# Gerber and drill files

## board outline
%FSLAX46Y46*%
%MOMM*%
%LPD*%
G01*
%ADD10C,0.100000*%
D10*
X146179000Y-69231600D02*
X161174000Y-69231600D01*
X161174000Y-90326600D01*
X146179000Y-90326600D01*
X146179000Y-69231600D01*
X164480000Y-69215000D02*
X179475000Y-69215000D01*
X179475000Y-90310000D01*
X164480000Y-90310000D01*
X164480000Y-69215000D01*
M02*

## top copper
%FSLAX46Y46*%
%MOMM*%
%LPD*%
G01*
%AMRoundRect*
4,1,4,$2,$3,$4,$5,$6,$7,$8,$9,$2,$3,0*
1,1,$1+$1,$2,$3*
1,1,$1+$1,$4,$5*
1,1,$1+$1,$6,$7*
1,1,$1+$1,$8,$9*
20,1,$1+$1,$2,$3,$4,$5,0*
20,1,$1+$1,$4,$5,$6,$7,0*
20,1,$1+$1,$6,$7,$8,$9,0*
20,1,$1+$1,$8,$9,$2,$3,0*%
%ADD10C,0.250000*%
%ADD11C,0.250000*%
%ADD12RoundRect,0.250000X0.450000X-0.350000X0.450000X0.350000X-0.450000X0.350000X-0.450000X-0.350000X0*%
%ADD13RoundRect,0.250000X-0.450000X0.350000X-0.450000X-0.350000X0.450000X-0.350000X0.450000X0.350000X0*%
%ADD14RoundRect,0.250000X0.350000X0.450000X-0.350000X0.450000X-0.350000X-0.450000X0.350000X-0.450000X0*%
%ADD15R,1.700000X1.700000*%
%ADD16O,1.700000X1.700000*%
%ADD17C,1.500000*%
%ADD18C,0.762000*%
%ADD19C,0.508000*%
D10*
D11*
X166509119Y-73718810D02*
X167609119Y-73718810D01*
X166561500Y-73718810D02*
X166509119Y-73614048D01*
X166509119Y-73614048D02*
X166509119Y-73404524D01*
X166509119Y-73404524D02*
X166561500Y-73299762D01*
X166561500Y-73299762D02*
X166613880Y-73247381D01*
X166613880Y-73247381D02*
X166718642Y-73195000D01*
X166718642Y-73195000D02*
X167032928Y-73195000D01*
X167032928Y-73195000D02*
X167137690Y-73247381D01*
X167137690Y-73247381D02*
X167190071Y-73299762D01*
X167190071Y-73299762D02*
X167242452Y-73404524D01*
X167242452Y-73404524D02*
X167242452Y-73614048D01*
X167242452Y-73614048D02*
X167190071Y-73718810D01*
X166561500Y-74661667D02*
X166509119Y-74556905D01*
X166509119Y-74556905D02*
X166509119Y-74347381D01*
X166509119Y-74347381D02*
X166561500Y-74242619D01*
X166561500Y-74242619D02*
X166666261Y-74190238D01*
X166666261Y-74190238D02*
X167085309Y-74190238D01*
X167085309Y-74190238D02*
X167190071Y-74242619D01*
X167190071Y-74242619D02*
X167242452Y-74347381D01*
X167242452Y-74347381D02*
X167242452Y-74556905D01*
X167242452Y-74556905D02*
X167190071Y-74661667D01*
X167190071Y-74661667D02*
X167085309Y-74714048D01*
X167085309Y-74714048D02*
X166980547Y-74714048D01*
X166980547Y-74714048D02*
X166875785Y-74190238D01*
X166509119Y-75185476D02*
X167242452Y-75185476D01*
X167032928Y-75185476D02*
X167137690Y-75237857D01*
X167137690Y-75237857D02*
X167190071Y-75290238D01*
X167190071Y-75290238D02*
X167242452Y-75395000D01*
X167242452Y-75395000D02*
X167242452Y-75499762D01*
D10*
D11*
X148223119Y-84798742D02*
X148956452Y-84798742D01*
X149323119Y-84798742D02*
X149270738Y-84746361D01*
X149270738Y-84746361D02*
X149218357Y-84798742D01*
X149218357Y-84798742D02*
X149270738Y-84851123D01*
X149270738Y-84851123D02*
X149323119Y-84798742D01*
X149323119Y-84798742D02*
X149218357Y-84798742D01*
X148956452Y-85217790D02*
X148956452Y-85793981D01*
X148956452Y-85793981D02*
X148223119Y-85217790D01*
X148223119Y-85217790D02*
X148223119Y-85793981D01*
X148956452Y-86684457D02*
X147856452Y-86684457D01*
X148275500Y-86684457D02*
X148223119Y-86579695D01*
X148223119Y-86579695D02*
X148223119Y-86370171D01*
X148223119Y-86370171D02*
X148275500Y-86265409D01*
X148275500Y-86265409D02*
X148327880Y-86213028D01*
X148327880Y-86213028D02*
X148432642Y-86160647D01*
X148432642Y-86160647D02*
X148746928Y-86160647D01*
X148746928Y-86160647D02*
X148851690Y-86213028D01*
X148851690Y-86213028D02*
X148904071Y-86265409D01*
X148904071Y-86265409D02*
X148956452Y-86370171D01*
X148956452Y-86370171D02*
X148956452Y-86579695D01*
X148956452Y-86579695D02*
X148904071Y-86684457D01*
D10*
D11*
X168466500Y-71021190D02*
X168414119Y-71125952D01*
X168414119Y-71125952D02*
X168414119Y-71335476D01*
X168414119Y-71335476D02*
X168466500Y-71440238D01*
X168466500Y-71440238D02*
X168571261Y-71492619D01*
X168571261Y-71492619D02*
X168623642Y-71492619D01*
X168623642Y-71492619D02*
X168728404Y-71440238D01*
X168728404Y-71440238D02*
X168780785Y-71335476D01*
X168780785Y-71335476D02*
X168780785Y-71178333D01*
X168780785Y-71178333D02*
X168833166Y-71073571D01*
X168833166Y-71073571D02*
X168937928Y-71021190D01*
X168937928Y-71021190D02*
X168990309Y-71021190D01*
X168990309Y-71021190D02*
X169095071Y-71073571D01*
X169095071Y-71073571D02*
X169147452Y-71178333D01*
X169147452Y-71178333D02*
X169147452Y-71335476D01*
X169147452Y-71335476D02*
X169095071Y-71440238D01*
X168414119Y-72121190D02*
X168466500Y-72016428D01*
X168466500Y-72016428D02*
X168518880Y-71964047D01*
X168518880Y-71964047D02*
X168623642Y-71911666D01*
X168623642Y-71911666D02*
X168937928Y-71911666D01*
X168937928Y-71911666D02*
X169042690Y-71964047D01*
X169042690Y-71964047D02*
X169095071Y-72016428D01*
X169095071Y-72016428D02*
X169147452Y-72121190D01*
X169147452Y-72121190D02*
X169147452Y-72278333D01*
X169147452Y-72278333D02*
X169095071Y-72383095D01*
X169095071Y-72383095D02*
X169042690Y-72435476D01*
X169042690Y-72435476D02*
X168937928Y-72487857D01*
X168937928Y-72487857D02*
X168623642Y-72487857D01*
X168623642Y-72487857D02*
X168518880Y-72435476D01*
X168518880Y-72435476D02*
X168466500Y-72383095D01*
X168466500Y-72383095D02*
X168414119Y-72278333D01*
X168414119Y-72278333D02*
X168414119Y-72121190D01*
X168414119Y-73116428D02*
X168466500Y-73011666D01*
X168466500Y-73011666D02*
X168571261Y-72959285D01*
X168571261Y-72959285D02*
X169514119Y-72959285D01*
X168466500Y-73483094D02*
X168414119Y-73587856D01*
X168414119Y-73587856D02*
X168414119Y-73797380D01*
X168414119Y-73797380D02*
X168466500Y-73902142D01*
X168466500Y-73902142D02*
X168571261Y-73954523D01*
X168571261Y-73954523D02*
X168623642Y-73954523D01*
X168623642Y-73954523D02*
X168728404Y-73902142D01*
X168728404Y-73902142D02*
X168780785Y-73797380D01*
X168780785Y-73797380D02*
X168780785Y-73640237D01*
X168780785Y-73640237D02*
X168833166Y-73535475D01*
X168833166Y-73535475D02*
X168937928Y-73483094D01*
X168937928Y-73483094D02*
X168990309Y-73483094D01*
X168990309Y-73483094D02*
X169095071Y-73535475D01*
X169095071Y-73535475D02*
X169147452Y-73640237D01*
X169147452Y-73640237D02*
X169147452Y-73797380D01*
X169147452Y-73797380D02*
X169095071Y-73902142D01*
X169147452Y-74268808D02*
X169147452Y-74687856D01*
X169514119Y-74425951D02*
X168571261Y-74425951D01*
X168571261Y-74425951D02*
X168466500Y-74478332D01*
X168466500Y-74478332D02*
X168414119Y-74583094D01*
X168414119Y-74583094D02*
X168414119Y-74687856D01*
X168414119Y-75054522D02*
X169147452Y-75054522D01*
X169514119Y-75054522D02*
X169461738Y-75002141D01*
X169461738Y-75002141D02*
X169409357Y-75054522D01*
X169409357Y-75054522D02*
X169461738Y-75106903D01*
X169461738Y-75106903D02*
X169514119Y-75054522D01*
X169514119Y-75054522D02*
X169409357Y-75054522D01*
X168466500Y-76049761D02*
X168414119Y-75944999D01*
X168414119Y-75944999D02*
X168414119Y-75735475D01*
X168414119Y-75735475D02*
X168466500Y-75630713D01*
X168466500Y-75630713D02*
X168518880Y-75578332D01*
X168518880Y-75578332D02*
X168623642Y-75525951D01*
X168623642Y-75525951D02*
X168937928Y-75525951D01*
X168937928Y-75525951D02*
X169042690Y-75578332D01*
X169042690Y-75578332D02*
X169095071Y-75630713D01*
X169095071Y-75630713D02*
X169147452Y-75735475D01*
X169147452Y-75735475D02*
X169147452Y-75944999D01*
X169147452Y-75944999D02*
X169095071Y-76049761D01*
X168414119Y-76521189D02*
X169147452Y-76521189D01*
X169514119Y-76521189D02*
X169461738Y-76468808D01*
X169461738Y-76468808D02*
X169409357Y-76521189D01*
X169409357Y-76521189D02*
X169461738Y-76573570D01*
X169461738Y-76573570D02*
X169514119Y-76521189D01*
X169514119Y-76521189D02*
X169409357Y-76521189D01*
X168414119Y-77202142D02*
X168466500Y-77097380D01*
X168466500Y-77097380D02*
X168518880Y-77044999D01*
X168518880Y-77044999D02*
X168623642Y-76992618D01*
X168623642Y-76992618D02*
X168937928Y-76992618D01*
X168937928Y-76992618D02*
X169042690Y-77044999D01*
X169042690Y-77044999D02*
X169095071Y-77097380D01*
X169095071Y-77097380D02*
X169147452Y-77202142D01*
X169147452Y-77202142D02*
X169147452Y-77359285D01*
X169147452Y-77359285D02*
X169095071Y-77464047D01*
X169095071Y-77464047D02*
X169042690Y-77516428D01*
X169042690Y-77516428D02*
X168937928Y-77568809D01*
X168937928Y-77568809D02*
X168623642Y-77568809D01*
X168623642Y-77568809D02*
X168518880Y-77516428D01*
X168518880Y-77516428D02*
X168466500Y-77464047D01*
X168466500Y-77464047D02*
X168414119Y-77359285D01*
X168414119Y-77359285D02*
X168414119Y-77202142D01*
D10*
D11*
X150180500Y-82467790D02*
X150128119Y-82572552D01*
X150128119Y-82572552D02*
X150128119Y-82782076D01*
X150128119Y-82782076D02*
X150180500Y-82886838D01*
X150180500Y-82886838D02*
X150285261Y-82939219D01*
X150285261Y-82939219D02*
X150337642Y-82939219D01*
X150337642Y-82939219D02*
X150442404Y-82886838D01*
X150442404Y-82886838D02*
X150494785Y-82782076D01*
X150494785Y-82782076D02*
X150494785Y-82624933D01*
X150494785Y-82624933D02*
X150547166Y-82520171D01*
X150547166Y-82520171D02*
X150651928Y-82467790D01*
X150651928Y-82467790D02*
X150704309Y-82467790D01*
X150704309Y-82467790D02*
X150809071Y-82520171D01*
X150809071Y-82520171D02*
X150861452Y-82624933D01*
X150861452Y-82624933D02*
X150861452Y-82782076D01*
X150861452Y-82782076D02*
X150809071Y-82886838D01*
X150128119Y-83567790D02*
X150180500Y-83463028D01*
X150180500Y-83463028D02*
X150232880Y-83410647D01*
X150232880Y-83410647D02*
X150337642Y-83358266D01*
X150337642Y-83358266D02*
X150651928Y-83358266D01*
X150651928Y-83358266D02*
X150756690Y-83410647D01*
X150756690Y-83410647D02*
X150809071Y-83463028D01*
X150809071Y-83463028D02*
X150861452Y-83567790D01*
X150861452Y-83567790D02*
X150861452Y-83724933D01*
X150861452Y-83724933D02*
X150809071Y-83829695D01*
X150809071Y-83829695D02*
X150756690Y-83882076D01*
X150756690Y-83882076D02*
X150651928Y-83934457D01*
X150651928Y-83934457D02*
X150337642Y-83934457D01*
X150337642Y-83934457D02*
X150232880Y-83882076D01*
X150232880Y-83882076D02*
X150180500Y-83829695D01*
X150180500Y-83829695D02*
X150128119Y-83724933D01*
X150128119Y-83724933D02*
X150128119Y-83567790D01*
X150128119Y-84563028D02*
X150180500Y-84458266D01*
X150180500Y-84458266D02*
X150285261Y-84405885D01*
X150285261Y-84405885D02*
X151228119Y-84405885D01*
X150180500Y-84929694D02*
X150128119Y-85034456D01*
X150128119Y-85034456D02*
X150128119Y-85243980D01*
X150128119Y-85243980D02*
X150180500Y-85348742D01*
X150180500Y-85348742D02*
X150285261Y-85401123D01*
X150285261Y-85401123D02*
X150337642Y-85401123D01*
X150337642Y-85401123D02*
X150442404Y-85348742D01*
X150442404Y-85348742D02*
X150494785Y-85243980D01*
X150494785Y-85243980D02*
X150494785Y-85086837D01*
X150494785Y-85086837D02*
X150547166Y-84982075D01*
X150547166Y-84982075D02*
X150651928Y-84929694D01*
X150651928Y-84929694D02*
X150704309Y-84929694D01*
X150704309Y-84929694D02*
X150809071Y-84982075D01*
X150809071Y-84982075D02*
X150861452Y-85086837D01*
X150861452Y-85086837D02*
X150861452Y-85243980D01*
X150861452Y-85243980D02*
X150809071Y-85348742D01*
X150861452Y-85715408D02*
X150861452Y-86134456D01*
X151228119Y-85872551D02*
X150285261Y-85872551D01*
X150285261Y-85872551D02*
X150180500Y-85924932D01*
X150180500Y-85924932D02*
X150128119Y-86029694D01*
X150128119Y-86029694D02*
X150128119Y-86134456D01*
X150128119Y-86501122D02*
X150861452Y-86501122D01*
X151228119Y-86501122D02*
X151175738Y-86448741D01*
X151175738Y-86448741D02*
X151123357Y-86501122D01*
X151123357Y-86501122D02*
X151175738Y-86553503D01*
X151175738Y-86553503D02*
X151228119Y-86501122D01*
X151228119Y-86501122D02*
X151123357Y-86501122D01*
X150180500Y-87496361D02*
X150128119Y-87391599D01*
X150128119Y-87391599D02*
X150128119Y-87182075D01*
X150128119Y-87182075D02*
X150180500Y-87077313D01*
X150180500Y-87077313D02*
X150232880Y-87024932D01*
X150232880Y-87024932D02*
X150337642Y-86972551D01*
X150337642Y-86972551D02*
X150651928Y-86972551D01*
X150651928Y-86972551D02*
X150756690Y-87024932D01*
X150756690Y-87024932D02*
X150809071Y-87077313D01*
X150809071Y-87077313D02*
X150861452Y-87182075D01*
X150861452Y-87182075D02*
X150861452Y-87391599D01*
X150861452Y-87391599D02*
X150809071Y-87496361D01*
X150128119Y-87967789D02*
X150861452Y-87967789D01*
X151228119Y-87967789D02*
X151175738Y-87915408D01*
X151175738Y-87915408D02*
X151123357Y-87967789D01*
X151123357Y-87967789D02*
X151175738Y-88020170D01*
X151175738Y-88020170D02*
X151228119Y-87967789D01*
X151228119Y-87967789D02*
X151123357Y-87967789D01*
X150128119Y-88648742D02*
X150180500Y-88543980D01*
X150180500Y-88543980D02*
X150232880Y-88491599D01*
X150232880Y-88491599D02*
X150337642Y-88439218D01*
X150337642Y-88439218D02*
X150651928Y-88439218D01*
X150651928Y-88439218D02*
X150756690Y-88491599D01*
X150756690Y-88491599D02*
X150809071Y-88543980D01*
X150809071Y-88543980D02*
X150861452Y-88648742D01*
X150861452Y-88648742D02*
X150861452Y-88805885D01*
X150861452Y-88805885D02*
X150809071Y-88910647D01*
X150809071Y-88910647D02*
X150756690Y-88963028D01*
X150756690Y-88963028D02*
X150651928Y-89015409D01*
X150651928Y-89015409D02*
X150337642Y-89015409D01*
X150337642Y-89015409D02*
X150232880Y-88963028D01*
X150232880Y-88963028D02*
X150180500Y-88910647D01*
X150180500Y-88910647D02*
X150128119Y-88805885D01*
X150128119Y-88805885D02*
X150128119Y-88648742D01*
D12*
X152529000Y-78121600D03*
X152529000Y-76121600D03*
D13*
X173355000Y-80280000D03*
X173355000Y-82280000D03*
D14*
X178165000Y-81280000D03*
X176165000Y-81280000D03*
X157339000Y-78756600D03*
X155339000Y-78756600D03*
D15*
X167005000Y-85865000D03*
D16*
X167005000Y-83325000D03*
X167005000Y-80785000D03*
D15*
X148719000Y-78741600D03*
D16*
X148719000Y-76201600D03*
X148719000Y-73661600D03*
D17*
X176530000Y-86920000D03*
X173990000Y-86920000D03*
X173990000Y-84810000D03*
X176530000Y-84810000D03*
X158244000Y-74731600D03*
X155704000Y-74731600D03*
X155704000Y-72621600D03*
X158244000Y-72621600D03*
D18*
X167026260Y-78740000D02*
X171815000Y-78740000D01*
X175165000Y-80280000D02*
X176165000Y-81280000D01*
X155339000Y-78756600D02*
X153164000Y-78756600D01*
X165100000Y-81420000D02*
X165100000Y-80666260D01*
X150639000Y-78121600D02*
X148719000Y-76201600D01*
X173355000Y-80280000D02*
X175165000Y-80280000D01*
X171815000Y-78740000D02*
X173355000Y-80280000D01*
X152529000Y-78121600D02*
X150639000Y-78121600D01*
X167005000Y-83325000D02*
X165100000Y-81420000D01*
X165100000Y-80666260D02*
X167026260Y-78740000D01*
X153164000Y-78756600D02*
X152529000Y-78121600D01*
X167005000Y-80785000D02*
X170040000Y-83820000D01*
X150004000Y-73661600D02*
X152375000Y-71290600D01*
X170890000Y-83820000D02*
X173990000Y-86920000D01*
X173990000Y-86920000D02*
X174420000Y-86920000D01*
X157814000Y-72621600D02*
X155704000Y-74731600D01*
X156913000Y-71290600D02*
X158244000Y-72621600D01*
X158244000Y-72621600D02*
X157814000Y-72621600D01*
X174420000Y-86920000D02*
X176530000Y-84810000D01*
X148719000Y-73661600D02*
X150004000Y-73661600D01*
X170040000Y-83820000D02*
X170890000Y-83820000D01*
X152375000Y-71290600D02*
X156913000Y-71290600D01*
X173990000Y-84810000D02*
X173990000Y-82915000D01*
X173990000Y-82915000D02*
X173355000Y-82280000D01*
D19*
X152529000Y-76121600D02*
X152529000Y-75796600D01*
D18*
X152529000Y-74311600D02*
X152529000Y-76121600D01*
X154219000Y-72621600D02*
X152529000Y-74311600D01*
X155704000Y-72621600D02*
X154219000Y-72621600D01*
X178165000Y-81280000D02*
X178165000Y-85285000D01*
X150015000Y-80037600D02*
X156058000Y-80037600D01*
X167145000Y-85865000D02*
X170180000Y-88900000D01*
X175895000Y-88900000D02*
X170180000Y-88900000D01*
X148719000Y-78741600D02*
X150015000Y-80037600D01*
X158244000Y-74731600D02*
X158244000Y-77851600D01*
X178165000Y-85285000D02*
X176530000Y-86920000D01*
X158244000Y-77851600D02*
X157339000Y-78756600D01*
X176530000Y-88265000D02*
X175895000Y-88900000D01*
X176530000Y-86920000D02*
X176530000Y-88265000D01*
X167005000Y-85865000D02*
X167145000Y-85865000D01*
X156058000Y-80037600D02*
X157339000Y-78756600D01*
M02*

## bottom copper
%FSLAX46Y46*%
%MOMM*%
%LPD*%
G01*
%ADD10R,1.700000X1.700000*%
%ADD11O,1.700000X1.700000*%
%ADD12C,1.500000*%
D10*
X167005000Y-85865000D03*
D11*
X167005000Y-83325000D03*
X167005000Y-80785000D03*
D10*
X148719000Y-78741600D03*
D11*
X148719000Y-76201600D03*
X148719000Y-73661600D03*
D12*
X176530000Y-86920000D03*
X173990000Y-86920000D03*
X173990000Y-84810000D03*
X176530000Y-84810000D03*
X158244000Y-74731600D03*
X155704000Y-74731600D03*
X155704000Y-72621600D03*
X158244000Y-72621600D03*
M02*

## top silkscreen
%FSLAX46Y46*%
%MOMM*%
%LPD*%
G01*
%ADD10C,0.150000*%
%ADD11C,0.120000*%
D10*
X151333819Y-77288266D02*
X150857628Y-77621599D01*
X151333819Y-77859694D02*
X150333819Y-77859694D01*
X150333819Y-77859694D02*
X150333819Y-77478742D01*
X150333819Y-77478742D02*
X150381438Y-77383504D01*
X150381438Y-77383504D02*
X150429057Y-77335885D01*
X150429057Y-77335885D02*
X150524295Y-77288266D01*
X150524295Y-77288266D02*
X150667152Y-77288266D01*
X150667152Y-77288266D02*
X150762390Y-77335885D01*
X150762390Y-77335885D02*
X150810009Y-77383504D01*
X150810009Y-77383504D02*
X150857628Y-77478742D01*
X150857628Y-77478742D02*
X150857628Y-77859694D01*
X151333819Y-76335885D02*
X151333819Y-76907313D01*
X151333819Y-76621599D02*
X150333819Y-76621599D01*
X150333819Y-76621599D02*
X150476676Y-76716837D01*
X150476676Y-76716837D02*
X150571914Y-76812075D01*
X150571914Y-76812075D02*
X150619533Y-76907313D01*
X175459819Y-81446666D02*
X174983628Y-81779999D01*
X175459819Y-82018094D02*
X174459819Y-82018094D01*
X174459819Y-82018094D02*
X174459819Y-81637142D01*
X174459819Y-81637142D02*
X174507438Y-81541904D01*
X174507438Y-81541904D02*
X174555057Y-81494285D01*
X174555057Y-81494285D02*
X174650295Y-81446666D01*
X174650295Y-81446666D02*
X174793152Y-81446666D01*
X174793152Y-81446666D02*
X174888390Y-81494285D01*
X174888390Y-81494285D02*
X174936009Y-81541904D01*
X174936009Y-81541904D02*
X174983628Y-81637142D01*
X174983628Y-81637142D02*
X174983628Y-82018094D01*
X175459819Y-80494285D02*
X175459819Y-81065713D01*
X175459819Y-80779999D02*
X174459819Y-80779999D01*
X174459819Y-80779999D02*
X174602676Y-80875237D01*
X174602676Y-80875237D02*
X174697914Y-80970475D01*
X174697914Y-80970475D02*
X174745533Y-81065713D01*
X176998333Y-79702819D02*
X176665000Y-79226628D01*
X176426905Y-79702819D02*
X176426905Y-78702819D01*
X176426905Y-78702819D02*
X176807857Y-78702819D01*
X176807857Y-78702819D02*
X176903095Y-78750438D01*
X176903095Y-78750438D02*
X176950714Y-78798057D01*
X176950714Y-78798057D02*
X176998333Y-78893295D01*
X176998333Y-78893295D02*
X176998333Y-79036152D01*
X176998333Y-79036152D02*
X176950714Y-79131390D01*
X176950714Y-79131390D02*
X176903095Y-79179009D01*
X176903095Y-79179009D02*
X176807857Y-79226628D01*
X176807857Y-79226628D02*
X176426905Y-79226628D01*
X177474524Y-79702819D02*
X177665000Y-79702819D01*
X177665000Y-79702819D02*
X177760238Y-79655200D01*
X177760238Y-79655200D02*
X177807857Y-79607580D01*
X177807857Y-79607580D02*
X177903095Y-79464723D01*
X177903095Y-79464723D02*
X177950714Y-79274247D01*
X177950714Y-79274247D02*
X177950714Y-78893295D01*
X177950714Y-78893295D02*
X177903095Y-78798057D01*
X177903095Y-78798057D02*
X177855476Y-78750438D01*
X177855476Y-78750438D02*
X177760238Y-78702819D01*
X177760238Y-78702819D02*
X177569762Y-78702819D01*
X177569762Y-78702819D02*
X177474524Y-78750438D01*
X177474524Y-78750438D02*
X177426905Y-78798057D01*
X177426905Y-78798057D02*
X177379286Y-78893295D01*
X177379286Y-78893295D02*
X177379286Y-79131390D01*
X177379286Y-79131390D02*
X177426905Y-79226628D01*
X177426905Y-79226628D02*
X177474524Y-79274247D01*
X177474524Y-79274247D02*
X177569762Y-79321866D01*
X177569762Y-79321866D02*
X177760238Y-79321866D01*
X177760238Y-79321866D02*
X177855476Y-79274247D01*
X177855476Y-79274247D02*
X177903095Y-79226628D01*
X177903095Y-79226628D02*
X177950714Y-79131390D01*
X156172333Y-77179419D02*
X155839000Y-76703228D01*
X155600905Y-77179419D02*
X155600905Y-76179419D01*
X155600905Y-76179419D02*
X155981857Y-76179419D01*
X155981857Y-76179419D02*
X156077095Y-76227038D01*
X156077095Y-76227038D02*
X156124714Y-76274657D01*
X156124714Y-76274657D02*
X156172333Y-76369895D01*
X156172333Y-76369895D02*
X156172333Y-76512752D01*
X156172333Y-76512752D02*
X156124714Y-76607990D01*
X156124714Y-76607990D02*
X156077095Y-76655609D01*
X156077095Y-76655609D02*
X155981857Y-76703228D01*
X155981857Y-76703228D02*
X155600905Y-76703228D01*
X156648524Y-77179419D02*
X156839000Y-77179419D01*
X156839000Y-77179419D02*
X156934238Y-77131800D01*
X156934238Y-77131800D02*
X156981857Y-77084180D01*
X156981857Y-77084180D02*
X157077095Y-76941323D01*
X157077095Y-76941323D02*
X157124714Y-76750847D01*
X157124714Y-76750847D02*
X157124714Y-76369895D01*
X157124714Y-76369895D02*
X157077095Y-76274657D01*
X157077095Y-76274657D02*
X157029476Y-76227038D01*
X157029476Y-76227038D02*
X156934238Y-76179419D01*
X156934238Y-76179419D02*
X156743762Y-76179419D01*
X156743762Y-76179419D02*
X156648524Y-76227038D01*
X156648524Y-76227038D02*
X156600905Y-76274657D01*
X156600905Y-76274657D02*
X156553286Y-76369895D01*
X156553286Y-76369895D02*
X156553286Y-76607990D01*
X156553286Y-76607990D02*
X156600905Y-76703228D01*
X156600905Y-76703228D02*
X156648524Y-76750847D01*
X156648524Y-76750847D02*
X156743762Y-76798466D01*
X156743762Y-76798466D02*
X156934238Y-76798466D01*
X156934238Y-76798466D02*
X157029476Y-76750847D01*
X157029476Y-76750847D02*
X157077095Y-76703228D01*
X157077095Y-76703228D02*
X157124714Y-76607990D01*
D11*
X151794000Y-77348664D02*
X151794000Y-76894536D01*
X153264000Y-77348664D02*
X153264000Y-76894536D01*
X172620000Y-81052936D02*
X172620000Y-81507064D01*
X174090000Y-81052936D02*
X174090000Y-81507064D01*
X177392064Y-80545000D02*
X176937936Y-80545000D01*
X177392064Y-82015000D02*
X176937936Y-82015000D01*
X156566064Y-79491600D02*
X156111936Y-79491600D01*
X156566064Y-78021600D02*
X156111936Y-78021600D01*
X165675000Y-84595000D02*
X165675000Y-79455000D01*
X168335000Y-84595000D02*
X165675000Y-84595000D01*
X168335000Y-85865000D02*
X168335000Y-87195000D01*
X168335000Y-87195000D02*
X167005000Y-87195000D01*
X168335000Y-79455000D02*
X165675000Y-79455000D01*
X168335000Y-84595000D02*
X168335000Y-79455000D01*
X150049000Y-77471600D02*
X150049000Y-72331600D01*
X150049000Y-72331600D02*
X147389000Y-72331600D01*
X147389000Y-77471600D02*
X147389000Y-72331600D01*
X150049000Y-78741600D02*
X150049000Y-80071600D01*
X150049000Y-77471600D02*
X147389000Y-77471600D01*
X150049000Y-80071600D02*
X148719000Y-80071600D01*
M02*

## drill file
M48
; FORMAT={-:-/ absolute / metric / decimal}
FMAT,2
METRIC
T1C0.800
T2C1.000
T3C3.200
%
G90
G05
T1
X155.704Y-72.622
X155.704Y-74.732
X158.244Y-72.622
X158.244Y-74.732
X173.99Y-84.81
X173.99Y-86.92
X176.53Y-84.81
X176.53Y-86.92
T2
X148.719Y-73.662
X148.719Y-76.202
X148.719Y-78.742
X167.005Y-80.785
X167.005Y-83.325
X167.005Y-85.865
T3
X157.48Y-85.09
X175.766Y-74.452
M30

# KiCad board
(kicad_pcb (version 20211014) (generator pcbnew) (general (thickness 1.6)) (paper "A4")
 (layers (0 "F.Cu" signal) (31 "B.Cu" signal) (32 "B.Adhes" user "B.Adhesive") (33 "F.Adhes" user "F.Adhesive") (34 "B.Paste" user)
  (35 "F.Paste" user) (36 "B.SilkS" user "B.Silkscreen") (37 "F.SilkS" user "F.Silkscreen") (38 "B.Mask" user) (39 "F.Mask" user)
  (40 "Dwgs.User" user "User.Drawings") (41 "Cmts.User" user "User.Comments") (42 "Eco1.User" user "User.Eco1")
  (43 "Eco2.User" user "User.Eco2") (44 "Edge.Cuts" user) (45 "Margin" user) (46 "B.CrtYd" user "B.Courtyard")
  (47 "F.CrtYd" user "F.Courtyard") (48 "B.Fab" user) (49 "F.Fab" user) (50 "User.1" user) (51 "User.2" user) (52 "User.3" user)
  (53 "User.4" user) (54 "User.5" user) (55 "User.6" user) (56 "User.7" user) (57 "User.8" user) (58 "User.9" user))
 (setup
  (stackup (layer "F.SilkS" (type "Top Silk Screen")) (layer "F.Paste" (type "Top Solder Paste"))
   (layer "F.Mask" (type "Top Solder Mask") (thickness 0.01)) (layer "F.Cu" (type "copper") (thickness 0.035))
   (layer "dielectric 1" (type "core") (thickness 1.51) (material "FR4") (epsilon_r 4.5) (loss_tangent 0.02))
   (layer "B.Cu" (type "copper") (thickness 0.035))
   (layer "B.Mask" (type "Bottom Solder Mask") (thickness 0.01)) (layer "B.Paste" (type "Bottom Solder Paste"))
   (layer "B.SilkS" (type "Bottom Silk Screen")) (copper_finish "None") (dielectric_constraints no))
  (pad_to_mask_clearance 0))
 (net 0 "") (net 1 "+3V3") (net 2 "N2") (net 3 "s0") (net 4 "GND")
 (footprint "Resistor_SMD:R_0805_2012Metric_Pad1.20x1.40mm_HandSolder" (layer "F.Cu") (at 152.529 77.1216 90)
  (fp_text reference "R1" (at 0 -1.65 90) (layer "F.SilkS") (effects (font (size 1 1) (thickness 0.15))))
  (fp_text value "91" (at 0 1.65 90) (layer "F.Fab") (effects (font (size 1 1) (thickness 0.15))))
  (fp_line (start -0.227064 -0.735) (end 0.227064 -0.735) (layer "F.SilkS") (width 0.12))
  (fp_line (start -0.227064 0.735) (end 0.227064 0.735) (layer "F.SilkS") (width 0.12))
  (pad "1" smd roundrect (at -1 0 90) (size 1.2 1.4) (layers "F.Cu" "F.Paste" "F.Mask") (roundrect_rratio 0.2083333333) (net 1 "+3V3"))
  (pad "2" smd roundrect (at 1 0 90) (size 1.2 1.4) (layers "F.Cu" "F.Paste" "F.Mask") (roundrect_rratio 0.2083333333) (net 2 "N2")))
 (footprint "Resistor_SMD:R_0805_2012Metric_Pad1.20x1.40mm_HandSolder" (layer "F.Cu") (at 173.355 81.28 -90)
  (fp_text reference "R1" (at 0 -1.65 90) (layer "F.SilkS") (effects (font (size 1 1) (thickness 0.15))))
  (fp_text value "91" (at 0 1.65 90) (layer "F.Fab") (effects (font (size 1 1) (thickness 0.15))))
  (fp_line (start -0.227064 0.735) (end 0.227064 0.735) (layer "F.SilkS") (width 0.12))
  (fp_line (start -0.227064 -0.735) (end 0.227064 -0.735) (layer "F.SilkS") (width 0.12))
  (pad "1" smd roundrect (at -1 0 270) (size 1.2 1.4) (layers "F.Cu" "F.Paste" "F.Mask") (roundrect_rratio 0.2083333333) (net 1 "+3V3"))
  (pad "2" smd roundrect (at 1 0 270) (size 1.2 1.4) (layers "F.Cu" "F.Paste" "F.Mask") (roundrect_rratio 0.2083333333) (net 2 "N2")))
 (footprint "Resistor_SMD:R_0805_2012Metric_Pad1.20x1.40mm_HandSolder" (layer "F.Cu") (at 177.165 81.28 180)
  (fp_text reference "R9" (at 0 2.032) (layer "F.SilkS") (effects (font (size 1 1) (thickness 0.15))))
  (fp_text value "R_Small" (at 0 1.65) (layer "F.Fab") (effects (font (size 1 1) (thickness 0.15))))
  (fp_line (start -0.227064 0.735) (end 0.227064 0.735) (layer "F.SilkS") (width 0.12))
  (fp_line (start -0.227064 -0.735) (end 0.227064 -0.735) (layer "F.SilkS") (width 0.12))
  (pad "1" smd roundrect (at -1 0 180) (size 1.2 1.4) (layers "F.Cu" "F.Paste" "F.Mask") (roundrect_rratio 0.2083333333) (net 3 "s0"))
  (pad "2" smd roundrect (at 1 0 180) (size 1.2 1.4) (layers "F.Cu" "F.Paste" "F.Mask") (roundrect_rratio 0.2083333333) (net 1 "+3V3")))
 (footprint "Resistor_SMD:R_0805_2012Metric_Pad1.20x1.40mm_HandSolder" (layer "F.Cu") (at 156.339 78.7566 180)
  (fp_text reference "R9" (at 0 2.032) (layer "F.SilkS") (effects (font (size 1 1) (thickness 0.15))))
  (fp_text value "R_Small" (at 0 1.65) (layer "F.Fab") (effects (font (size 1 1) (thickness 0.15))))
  (fp_line (start -0.227064 -0.735) (end 0.227064 -0.735) (layer "F.SilkS") (width 0.12))
  (fp_line (start -0.227064 0.735) (end 0.227064 0.735) (layer "F.SilkS") (width 0.12))
  (pad "1" smd roundrect (at -1 0 180) (size 1.2 1.4) (layers "F.Cu" "F.Paste" "F.Mask") (roundrect_rratio 0.2083333333) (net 3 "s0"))
  (pad "2" smd roundrect (at 1 0 180) (size 1.2 1.4) (layers "F.Cu" "F.Paste" "F.Mask") (roundrect_rratio 0.2083333333) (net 1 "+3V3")))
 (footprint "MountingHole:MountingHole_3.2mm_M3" (layer "F.Cu") (at 175.766 74.452)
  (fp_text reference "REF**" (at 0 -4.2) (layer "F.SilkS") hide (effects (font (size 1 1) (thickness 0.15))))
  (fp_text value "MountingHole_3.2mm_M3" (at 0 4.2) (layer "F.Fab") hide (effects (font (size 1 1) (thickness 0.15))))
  (pad "" np_thru_hole circle (at 0 0) (size 3.2 3.2) (drill 3.2) (layers F&B.Cu *.Mask)))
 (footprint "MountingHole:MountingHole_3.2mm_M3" (layer "F.Cu") (at 157.48 85.09 180)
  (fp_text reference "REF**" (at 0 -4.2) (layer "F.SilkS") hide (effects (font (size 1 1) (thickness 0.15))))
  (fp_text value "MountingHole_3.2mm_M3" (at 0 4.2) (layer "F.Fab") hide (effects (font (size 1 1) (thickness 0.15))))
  (pad "" np_thru_hole circle (at 0 0 180) (size 3.2 3.2) (drill 3.2) (layers *.Cu *.Mask)))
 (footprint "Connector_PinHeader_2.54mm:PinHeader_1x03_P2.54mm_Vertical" (layer "F.Cu") (at 167.005 85.865 180)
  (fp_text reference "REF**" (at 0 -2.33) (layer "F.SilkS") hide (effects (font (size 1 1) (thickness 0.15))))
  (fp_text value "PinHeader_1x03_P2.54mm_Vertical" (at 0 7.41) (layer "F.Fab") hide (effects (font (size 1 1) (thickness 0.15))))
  (fp_line (start 1.33 1.27) (end 1.33 6.41) (layer "F.SilkS") (width 0.12))
  (fp_line (start -1.33 1.27) (end 1.33 1.27) (layer "F.SilkS") (width 0.12))
  (fp_line (start -1.33 0) (end -1.33 -1.33) (layer "F.SilkS") (width 0.12))
  (fp_line (start -1.33 -1.33) (end 0 -1.33) (layer "F.SilkS") (width 0.12))
  (fp_line (start -1.33 6.41) (end 1.33 6.41) (layer "F.SilkS") (width 0.12))
  (fp_line (start -1.33 1.27) (end -1.33 6.41) (layer "F.SilkS") (width 0.12))
  (pad "1" thru_hole rect (at 0 0 180) (size 1.7 1.7) (drill 1) (layers *.Cu *.Mask) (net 3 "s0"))
  (pad "2" thru_hole oval (at 0 2.54 180) (size 1.7 1.7) (drill 1) (layers *.Cu *.Mask) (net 1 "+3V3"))
  (pad "3" thru_hole oval (at 0 5.08 180) (size 1.7 1.7) (drill 1) (layers *.Cu *.Mask) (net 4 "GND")))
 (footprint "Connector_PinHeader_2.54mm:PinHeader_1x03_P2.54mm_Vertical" (layer "F.Cu") (at 148.719 78.7416 180)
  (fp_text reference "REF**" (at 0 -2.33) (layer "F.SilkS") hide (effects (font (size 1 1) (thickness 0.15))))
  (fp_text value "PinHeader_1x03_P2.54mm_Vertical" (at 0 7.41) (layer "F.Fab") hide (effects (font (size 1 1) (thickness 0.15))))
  (fp_line (start -1.33 1.27) (end -1.33 6.41) (layer "F.SilkS") (width 0.12))
  (fp_line (start -1.33 6.41) (end 1.33 6.41) (layer "F.SilkS") (width 0.12))
  (fp_line (start 1.33 1.27) (end 1.33 6.41) (layer "F.SilkS") (width 0.12))
  (fp_line (start -1.33 0) (end -1.33 -1.33) (layer "F.SilkS") (width 0.12))
  (fp_line (start -1.33 1.27) (end 1.33 1.27) (layer "F.SilkS") (width 0.12))
  (fp_line (start -1.33 -1.33) (end 0 -1.33) (layer "F.SilkS") (width 0.12))
  (pad "1" thru_hole rect (at 0 0 180) (size 1.7 1.7) (drill 1) (layers *.Cu *.Mask) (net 3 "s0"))
  (pad "2" thru_hole oval (at 0 2.54 180) (size 1.7 1.7) (drill 1) (layers *.Cu *.Mask) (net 1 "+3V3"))
  (pad "3" thru_hole oval (at 0 5.08 180) (size 1.7 1.7) (drill 1) (layers *.Cu *.Mask) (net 4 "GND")))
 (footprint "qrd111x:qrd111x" (layer "B.Cu") (at 175.26 85.865 90)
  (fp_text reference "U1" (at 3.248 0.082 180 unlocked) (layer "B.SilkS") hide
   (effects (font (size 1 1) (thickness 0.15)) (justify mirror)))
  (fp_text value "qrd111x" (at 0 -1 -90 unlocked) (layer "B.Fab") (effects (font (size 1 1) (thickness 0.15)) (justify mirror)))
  (pad "1" thru_hole circle (at -1.055 1.27 270) (size 1.5 1.5) (drill 0.8) (layers *.Cu *.Mask) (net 3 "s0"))
  (pad "2" thru_hole circle (at -1.055 -1.27 270) (size 1.5 1.5) (drill 0.8) (layers *.Cu *.Mask) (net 4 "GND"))
  (pad "3" thru_hole circle (at 1.055 -1.27 270) (size 1.5 1.5) (drill 0.8) (layers *.Cu *.Mask) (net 2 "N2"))
  (pad "4" thru_hole circle (at 1.055 1.27 270) (size 1.5 1.5) (drill 0.8) (layers *.Cu *.Mask) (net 4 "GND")))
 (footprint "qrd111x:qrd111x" (layer "B.Cu") (at 156.974 73.6766 90)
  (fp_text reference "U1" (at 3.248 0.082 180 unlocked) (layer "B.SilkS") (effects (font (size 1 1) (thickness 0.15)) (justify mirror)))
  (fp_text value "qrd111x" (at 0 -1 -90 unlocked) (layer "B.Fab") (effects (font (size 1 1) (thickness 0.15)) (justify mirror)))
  (pad "1" thru_hole circle (at -1.055 1.27 270) (size 1.5 1.5) (drill 0.8) (layers *.Cu *.Mask) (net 3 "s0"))
  (pad "2" thru_hole circle (at -1.055 -1.27 270) (size 1.5 1.5) (drill 0.8) (layers *.Cu *.Mask) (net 4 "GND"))
  (pad "3" thru_hole circle (at 1.055 -1.27 270) (size 1.5 1.5) (drill 0.8) (layers *.Cu *.Mask) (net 2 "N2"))
  (pad "4" thru_hole circle (at 1.055 1.27 270) (size 1.5 1.5) (drill 0.8) (layers *.Cu *.Mask) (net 4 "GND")))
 (gr_rect (start 146.179 69.2316) (end 161.174 90.3266) (layer "Edge.Cuts") (width 0.1) (fill none))
 (gr_rect (start 179.475 90.31) (end 164.48 69.215) (layer "Edge.Cuts") (width 0.1) (fill none))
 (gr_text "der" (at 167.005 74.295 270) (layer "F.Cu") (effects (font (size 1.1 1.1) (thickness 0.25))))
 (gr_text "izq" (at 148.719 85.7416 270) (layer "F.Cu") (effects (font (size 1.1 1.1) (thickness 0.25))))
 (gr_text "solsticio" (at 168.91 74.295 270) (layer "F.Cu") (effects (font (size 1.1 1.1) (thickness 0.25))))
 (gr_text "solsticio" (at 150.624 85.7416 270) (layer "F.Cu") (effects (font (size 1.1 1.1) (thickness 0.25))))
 (segment (start 167.02626 78.74) (end 171.815 78.74) (width 0.762) (layer "F.Cu") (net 1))
 (segment (start 175.165 80.28) (end 176.165 81.28) (width 0.762) (layer "F.Cu") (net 1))
 (segment (start 155.339 78.7566) (end 153.164 78.7566) (width 0.762) (layer "F.Cu") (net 1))
 (segment (start 165.1 81.42) (end 165.1 80.66626) (width 0.762) (layer "F.Cu") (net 1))
 (segment (start 150.639 78.1216) (end 148.719 76.2016) (width 0.762) (layer "F.Cu") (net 1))
 (segment (start 173.355 80.28) (end 175.165 80.28) (width 0.762) (layer "F.Cu") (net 1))
 (segment (start 171.815 78.74) (end 173.355 80.28) (width 0.762) (layer "F.Cu") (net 1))
 (segment (start 152.529 78.1216) (end 150.639 78.1216) (width 0.762) (layer "F.Cu") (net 1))
 (segment (start 167.005 83.325) (end 165.1 81.42) (width 0.762) (layer "F.Cu") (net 1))
 (segment (start 165.1 80.66626) (end 167.02626 78.74) (width 0.762) (layer "F.Cu") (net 1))
 (segment (start 153.164 78.7566) (end 152.529 78.1216) (width 0.762) (layer "F.Cu") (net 1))
 (segment (start 167.005 80.785) (end 170.04 83.82) (width 0.762) (layer "F.Cu") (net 4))
 (segment (start 150.004 73.6616) (end 152.375 71.2906) (width 0.762) (layer "F.Cu") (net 4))
 (segment (start 170.89 83.82) (end 173.99 86.92) (width 0.762) (layer "F.Cu") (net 4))
 (segment (start 173.99 86.92) (end 174.42 86.92) (width 0.762) (layer "F.Cu") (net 4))
 (segment (start 157.814 72.6216) (end 155.704 74.7316) (width 0.762) (layer "F.Cu") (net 4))
 (segment (start 156.913 71.2906) (end 158.244 72.6216) (width 0.762) (layer "F.Cu") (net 4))
 (segment (start 158.244 72.6216) (end 157.814 72.6216) (width 0.762) (layer "F.Cu") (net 4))
 (segment (start 174.42 86.92) (end 176.53 84.81) (width 0.762) (layer "F.Cu") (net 4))
 (segment (start 148.719 73.6616) (end 150.004 73.6616) (width 0.762) (layer "F.Cu") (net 4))
 (segment (start 170.04 83.82) (end 170.89 83.82) (width 0.762) (layer "F.Cu") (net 4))
 (segment (start 152.375 71.2906) (end 156.913 71.2906) (width 0.762) (layer "F.Cu") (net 4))
 (segment (start 173.99 84.81) (end 173.99 82.915) (width 0.762) (layer "F.Cu") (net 2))
 (segment (start 173.99 82.915) (end 173.355 82.28) (width 0.762) (layer "F.Cu") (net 2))
 (segment (start 152.529 76.1216) (end 152.529 75.7966) (width 0.508) (layer "F.Cu") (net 2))
 (segment (start 152.529 74.3116) (end 152.529 76.1216) (width 0.762) (layer "F.Cu") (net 2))
 (segment (start 154.219 72.6216) (end 152.529 74.3116) (width 0.762) (layer "F.Cu") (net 2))
 (segment (start 155.704 72.6216) (end 154.219 72.6216) (width 0.762) (layer "F.Cu") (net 2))
 (segment (start 178.165 81.28) (end 178.165 85.285) (width 0.762) (layer "F.Cu") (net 3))
 (segment (start 150.015 80.0376) (end 156.058 80.0376) (width 0.762) (layer "F.Cu") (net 3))
 (segment (start 167.145 85.865) (end 170.18 88.9) (width 0.762) (layer "F.Cu") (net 3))
 (segment (start 175.895 88.9) (end 170.18 88.9) (width 0.762) (layer "F.Cu") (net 3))
 (segment (start 148.719 78.7416) (end 150.015 80.0376) (width 0.762) (layer "F.Cu") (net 3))
 (segment (start 158.244 74.7316) (end 158.244 77.8516) (width 0.762) (layer "F.Cu") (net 3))
 (segment (start 178.165 85.285) (end 176.53 86.92) (width 0.762) (layer "F.Cu") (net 3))
 (segment (start 158.244 77.8516) (end 157.339 78.7566) (width 0.762) (layer "F.Cu") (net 3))
 (segment (start 176.53 88.265) (end 175.895 88.9) (width 0.762) (layer "F.Cu") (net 3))
 (segment (start 176.53 86.92) (end 176.53 88.265) (width 0.762) (layer "F.Cu") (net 3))
 (segment (start 167.005 85.865) (end 167.145 85.865) (width 0.762) (layer "F.Cu") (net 3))
 (segment (start 156.058 80.0376) (end 157.339 78.7566) (width 0.762) (layer "F.Cu") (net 3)))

